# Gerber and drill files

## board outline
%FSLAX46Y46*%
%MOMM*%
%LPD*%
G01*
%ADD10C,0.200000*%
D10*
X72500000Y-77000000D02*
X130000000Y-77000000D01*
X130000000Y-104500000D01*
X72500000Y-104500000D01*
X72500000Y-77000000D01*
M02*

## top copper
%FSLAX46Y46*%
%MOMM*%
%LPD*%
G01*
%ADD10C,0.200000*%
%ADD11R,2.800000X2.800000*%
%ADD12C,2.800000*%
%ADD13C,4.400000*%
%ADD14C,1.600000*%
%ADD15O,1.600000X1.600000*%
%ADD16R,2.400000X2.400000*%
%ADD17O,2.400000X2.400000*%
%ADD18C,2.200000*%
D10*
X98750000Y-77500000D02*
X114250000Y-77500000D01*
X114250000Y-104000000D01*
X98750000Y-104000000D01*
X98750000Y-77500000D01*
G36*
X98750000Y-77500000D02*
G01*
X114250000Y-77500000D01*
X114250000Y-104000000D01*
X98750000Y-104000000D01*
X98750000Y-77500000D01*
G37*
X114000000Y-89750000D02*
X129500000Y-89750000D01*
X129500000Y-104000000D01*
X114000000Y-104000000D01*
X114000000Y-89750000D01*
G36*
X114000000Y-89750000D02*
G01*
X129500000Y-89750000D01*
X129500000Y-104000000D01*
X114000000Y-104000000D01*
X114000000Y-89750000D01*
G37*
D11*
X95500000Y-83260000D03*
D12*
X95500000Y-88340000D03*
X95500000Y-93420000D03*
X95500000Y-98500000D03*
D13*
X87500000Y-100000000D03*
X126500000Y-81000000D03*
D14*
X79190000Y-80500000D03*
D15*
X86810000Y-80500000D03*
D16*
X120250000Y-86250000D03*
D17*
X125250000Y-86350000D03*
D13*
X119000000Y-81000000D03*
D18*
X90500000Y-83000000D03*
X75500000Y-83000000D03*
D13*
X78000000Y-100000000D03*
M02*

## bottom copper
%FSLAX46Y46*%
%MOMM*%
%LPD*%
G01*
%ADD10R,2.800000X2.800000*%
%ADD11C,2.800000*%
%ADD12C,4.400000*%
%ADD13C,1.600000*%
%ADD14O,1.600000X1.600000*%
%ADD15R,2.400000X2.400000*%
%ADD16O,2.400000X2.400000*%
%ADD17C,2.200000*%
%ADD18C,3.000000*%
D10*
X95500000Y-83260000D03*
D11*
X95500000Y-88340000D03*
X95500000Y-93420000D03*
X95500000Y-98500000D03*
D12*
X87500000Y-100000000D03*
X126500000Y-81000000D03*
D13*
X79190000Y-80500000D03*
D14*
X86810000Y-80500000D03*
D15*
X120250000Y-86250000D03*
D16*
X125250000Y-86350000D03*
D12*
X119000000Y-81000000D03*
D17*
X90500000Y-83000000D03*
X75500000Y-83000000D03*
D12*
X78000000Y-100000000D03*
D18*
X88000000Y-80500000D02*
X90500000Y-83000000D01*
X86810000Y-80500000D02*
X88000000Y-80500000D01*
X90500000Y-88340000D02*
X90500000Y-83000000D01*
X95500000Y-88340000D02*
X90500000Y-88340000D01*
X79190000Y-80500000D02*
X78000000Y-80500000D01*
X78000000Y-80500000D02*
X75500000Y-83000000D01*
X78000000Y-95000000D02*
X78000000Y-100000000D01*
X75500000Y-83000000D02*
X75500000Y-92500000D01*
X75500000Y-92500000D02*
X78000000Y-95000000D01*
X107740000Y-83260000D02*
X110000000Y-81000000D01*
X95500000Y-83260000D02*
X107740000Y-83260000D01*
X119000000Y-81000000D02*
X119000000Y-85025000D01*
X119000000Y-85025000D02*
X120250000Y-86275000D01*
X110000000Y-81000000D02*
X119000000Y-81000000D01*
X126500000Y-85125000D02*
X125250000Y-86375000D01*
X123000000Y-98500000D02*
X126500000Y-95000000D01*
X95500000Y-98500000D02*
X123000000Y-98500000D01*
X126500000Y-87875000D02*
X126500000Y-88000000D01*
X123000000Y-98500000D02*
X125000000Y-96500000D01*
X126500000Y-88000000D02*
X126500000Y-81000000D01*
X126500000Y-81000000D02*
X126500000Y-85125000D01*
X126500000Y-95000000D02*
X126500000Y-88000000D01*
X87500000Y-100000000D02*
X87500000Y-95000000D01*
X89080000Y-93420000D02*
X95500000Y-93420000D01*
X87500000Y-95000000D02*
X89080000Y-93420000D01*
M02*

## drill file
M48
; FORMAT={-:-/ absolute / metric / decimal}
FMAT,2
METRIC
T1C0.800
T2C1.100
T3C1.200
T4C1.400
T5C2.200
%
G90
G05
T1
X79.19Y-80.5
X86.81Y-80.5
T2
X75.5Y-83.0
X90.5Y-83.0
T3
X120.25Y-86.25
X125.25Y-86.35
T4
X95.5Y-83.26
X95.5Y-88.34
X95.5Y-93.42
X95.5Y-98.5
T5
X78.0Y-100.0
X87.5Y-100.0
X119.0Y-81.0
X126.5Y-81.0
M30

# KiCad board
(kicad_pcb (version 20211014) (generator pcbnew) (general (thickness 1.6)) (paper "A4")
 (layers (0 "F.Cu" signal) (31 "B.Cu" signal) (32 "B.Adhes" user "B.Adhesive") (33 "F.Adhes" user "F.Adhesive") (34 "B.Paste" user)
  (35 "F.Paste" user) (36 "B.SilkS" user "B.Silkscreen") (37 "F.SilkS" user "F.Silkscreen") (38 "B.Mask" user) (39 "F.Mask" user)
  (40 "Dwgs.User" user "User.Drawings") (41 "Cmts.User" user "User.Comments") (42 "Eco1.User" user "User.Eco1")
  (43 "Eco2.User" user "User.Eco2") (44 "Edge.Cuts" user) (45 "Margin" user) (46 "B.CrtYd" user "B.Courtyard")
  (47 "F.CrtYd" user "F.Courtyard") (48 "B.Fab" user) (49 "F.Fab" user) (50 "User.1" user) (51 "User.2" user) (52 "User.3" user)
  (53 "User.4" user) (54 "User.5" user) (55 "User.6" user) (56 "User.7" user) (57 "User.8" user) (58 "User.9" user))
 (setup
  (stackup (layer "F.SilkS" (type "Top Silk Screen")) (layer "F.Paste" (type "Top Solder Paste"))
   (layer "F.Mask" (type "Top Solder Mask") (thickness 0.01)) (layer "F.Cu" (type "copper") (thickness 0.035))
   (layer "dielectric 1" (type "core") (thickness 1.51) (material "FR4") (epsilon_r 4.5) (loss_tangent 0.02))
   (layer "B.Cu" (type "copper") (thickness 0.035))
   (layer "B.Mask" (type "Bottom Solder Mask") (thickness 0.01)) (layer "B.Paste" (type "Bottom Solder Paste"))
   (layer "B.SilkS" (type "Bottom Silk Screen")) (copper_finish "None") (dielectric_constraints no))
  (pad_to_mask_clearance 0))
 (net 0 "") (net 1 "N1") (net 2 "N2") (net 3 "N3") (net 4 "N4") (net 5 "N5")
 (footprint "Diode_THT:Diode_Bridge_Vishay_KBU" (layer "F.Cu") (at 95.5 98.5 90)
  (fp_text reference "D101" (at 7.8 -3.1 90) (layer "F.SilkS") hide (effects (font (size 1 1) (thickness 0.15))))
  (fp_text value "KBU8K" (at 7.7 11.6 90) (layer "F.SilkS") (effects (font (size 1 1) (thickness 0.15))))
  (pad "1" thru_hole rect (at 15.24 0 90) (size 2.8 2.8) (drill 1.4) (layers *.Cu *.Mask) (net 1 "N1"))
  (pad "2" thru_hole circle (at 10.16 0 90) (size 2.8 2.8) (drill 1.4) (layers *.Cu *.Mask) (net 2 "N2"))
  (pad "3" thru_hole circle (at 5.08 0 90) (size 2.8 2.8) (drill 1.4) (layers *.Cu *.Mask) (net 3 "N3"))
  (pad "4" thru_hole circle (at 0 0 90) (size 2.8 2.8) (drill 1.4) (layers *.Cu *.Mask) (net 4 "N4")))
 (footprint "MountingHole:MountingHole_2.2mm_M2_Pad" (layer "F.Cu") (at 87.5 100)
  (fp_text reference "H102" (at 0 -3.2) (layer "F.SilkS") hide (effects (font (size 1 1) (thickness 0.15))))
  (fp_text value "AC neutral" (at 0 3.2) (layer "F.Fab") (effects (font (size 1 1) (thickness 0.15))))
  (pad "1" thru_hole circle (at 0 0) (size 4.4 4.4) (drill 2.2) (layers *.Cu *.Mask) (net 3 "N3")))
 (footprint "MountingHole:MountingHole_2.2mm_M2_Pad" (layer "F.Cu") (at 126.5 81 180)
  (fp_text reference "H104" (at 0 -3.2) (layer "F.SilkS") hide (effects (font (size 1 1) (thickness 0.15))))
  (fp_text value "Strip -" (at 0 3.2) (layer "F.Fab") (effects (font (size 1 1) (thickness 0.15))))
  (pad "1" thru_hole circle (at 0 0 180) (size 4.4 4.4) (drill 2.2) (layers *.Cu *.Mask) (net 4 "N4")))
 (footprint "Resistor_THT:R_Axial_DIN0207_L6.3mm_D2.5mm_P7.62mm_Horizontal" (layer "F.Cu") (at 79.19 80.5)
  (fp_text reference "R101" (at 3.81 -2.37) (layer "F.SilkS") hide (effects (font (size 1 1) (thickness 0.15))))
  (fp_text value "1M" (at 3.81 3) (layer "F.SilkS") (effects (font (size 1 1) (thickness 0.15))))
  (pad "1" thru_hole circle (at 0 0) (size 1.6 1.6) (drill 0.8) (layers *.Cu *.Mask) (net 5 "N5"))
  (pad "2" thru_hole oval (at 7.62 0) (size 1.6 1.6) (drill 0.8) (layers *.Cu *.Mask) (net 2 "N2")))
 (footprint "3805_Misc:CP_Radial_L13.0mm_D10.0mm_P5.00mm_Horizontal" (layer "F.Cu") (at 122.75 101.65 90)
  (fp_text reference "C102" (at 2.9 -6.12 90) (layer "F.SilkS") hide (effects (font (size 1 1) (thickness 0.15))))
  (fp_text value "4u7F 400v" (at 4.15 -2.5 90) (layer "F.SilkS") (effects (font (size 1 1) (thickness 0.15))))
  (pad "1" thru_hole rect (at 15.4 -2.5 90) (size 2.4 2.4) (drill 1.2) (layers *.Cu *.Mask) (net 1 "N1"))
  (pad "2" thru_hole oval (at 15.3 2.5 90) (size 2.4 2.4) (drill 1.2) (layers *.Cu *.Mask) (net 4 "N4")))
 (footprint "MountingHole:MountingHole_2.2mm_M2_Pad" (layer "F.Cu") (at 119 81)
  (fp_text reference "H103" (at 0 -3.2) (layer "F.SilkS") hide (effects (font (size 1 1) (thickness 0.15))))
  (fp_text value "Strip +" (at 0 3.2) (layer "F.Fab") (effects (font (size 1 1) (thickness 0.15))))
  (pad "1" thru_hole circle (at 0 0) (size 4.4 4.4) (drill 2.2) (layers *.Cu *.Mask) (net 1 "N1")))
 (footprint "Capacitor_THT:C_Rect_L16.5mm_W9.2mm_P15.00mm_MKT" (layer "F.Cu") (at 90.5 83 180)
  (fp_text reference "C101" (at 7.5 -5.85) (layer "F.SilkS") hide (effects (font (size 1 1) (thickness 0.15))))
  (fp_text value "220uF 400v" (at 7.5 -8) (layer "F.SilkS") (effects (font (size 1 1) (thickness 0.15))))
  (pad "1" thru_hole circle (at 0 0 180) (size 2.2 2.2) (drill 1.1) (layers *.Cu *.Mask) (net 2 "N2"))
  (pad "2" thru_hole circle (at 15 0 180) (size 2.2 2.2) (drill 1.1) (layers *.Cu *.Mask) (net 5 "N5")))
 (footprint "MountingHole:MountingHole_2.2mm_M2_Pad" (layer "F.Cu") (at 78 100)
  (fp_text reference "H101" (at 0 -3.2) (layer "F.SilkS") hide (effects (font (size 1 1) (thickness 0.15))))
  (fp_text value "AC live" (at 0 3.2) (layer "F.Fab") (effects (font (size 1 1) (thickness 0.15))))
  (pad "1" thru_hole circle (at 0 0) (size 4.4 4.4) (drill 2.2) (layers *.Cu *.Mask) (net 5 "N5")))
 (gr_rect (start 98.75 77.5) (end 114.25 104) (layer "F.Cu") (width 0.2) (fill solid))
 (gr_rect (start 114 89.75) (end 129.5 104) (layer "F.Cu") (width 0.2) (fill solid))
 (gr_rect (start 72.5 77) (end 130 104.5) (layer "Edge.Cuts") (width 0.2) (fill none))
 (segment (start 88 80.5) (end 90.5 83) (width 3) (layer "B.Cu") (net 2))
 (segment (start 86.81 80.5) (end 88 80.5) (width 3) (layer "B.Cu") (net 2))
 (segment (start 90.5 88.34) (end 90.5 83) (width 3) (layer "B.Cu") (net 2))
 (segment (start 95.5 88.34) (end 90.5 88.34) (width 3) (layer "B.Cu") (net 2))
 (segment (start 79.19 80.5) (end 78 80.5) (width 3) (layer "B.Cu") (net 5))
 (segment (start 78 80.5) (end 75.5 83) (width 3) (layer "B.Cu") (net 5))
 (segment (start 78 95) (end 78 100) (width 3) (layer "B.Cu") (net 5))
 (segment (start 75.5 83) (end 75.5 92.5) (width 3) (layer "B.Cu") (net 5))
 (segment (start 75.5 92.5) (end 78 95) (width 3) (layer "B.Cu") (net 5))
 (segment (start 107.74 83.26) (end 110 81) (width 3) (layer "B.Cu") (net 1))
 (segment (start 95.5 83.26) (end 107.74 83.26) (width 3) (layer "B.Cu") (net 1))
 (segment (start 119 81) (end 119 85.025) (width 3) (layer "B.Cu") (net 1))
 (segment (start 119 85.025) (end 120.25 86.275) (width 3) (layer "B.Cu") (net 1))
 (segment (start 110 81) (end 119 81) (width 3) (layer "B.Cu") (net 1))
 (segment (start 126.5 85.125) (end 125.25 86.375) (width 3) (layer "B.Cu") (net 4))
 (segment (start 123 98.5) (end 126.5 95) (width 3) (layer "B.Cu") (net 4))
 (segment (start 95.5 98.5) (end 123 98.5) (width 3) (layer "B.Cu") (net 4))
 (segment (start 126.5 87.875) (end 126.5 88) (width 3) (layer "B.Cu") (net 4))
 (segment (start 123 98.5) (end 125 96.5) (width 3) (layer "B.Cu") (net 4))
 (segment (start 126.5 88) (end 126.5 81) (width 3) (layer "B.Cu") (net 4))
 (segment (start 126.5 81) (end 126.5 85.125) (width 3) (layer "B.Cu") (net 4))
 (segment (start 126.5 95) (end 126.5 88) (width 3) (layer "B.Cu") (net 4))
 (segment (start 87.5 100) (end 87.5 95) (width 3) (layer "B.Cu") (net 3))
 (segment (start 89.08 93.42) (end 95.5 93.42) (width 3) (layer "B.Cu") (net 3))
 (segment (start 87.5 95) (end 89.08 93.42) (width 3) (layer "B.Cu") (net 3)))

